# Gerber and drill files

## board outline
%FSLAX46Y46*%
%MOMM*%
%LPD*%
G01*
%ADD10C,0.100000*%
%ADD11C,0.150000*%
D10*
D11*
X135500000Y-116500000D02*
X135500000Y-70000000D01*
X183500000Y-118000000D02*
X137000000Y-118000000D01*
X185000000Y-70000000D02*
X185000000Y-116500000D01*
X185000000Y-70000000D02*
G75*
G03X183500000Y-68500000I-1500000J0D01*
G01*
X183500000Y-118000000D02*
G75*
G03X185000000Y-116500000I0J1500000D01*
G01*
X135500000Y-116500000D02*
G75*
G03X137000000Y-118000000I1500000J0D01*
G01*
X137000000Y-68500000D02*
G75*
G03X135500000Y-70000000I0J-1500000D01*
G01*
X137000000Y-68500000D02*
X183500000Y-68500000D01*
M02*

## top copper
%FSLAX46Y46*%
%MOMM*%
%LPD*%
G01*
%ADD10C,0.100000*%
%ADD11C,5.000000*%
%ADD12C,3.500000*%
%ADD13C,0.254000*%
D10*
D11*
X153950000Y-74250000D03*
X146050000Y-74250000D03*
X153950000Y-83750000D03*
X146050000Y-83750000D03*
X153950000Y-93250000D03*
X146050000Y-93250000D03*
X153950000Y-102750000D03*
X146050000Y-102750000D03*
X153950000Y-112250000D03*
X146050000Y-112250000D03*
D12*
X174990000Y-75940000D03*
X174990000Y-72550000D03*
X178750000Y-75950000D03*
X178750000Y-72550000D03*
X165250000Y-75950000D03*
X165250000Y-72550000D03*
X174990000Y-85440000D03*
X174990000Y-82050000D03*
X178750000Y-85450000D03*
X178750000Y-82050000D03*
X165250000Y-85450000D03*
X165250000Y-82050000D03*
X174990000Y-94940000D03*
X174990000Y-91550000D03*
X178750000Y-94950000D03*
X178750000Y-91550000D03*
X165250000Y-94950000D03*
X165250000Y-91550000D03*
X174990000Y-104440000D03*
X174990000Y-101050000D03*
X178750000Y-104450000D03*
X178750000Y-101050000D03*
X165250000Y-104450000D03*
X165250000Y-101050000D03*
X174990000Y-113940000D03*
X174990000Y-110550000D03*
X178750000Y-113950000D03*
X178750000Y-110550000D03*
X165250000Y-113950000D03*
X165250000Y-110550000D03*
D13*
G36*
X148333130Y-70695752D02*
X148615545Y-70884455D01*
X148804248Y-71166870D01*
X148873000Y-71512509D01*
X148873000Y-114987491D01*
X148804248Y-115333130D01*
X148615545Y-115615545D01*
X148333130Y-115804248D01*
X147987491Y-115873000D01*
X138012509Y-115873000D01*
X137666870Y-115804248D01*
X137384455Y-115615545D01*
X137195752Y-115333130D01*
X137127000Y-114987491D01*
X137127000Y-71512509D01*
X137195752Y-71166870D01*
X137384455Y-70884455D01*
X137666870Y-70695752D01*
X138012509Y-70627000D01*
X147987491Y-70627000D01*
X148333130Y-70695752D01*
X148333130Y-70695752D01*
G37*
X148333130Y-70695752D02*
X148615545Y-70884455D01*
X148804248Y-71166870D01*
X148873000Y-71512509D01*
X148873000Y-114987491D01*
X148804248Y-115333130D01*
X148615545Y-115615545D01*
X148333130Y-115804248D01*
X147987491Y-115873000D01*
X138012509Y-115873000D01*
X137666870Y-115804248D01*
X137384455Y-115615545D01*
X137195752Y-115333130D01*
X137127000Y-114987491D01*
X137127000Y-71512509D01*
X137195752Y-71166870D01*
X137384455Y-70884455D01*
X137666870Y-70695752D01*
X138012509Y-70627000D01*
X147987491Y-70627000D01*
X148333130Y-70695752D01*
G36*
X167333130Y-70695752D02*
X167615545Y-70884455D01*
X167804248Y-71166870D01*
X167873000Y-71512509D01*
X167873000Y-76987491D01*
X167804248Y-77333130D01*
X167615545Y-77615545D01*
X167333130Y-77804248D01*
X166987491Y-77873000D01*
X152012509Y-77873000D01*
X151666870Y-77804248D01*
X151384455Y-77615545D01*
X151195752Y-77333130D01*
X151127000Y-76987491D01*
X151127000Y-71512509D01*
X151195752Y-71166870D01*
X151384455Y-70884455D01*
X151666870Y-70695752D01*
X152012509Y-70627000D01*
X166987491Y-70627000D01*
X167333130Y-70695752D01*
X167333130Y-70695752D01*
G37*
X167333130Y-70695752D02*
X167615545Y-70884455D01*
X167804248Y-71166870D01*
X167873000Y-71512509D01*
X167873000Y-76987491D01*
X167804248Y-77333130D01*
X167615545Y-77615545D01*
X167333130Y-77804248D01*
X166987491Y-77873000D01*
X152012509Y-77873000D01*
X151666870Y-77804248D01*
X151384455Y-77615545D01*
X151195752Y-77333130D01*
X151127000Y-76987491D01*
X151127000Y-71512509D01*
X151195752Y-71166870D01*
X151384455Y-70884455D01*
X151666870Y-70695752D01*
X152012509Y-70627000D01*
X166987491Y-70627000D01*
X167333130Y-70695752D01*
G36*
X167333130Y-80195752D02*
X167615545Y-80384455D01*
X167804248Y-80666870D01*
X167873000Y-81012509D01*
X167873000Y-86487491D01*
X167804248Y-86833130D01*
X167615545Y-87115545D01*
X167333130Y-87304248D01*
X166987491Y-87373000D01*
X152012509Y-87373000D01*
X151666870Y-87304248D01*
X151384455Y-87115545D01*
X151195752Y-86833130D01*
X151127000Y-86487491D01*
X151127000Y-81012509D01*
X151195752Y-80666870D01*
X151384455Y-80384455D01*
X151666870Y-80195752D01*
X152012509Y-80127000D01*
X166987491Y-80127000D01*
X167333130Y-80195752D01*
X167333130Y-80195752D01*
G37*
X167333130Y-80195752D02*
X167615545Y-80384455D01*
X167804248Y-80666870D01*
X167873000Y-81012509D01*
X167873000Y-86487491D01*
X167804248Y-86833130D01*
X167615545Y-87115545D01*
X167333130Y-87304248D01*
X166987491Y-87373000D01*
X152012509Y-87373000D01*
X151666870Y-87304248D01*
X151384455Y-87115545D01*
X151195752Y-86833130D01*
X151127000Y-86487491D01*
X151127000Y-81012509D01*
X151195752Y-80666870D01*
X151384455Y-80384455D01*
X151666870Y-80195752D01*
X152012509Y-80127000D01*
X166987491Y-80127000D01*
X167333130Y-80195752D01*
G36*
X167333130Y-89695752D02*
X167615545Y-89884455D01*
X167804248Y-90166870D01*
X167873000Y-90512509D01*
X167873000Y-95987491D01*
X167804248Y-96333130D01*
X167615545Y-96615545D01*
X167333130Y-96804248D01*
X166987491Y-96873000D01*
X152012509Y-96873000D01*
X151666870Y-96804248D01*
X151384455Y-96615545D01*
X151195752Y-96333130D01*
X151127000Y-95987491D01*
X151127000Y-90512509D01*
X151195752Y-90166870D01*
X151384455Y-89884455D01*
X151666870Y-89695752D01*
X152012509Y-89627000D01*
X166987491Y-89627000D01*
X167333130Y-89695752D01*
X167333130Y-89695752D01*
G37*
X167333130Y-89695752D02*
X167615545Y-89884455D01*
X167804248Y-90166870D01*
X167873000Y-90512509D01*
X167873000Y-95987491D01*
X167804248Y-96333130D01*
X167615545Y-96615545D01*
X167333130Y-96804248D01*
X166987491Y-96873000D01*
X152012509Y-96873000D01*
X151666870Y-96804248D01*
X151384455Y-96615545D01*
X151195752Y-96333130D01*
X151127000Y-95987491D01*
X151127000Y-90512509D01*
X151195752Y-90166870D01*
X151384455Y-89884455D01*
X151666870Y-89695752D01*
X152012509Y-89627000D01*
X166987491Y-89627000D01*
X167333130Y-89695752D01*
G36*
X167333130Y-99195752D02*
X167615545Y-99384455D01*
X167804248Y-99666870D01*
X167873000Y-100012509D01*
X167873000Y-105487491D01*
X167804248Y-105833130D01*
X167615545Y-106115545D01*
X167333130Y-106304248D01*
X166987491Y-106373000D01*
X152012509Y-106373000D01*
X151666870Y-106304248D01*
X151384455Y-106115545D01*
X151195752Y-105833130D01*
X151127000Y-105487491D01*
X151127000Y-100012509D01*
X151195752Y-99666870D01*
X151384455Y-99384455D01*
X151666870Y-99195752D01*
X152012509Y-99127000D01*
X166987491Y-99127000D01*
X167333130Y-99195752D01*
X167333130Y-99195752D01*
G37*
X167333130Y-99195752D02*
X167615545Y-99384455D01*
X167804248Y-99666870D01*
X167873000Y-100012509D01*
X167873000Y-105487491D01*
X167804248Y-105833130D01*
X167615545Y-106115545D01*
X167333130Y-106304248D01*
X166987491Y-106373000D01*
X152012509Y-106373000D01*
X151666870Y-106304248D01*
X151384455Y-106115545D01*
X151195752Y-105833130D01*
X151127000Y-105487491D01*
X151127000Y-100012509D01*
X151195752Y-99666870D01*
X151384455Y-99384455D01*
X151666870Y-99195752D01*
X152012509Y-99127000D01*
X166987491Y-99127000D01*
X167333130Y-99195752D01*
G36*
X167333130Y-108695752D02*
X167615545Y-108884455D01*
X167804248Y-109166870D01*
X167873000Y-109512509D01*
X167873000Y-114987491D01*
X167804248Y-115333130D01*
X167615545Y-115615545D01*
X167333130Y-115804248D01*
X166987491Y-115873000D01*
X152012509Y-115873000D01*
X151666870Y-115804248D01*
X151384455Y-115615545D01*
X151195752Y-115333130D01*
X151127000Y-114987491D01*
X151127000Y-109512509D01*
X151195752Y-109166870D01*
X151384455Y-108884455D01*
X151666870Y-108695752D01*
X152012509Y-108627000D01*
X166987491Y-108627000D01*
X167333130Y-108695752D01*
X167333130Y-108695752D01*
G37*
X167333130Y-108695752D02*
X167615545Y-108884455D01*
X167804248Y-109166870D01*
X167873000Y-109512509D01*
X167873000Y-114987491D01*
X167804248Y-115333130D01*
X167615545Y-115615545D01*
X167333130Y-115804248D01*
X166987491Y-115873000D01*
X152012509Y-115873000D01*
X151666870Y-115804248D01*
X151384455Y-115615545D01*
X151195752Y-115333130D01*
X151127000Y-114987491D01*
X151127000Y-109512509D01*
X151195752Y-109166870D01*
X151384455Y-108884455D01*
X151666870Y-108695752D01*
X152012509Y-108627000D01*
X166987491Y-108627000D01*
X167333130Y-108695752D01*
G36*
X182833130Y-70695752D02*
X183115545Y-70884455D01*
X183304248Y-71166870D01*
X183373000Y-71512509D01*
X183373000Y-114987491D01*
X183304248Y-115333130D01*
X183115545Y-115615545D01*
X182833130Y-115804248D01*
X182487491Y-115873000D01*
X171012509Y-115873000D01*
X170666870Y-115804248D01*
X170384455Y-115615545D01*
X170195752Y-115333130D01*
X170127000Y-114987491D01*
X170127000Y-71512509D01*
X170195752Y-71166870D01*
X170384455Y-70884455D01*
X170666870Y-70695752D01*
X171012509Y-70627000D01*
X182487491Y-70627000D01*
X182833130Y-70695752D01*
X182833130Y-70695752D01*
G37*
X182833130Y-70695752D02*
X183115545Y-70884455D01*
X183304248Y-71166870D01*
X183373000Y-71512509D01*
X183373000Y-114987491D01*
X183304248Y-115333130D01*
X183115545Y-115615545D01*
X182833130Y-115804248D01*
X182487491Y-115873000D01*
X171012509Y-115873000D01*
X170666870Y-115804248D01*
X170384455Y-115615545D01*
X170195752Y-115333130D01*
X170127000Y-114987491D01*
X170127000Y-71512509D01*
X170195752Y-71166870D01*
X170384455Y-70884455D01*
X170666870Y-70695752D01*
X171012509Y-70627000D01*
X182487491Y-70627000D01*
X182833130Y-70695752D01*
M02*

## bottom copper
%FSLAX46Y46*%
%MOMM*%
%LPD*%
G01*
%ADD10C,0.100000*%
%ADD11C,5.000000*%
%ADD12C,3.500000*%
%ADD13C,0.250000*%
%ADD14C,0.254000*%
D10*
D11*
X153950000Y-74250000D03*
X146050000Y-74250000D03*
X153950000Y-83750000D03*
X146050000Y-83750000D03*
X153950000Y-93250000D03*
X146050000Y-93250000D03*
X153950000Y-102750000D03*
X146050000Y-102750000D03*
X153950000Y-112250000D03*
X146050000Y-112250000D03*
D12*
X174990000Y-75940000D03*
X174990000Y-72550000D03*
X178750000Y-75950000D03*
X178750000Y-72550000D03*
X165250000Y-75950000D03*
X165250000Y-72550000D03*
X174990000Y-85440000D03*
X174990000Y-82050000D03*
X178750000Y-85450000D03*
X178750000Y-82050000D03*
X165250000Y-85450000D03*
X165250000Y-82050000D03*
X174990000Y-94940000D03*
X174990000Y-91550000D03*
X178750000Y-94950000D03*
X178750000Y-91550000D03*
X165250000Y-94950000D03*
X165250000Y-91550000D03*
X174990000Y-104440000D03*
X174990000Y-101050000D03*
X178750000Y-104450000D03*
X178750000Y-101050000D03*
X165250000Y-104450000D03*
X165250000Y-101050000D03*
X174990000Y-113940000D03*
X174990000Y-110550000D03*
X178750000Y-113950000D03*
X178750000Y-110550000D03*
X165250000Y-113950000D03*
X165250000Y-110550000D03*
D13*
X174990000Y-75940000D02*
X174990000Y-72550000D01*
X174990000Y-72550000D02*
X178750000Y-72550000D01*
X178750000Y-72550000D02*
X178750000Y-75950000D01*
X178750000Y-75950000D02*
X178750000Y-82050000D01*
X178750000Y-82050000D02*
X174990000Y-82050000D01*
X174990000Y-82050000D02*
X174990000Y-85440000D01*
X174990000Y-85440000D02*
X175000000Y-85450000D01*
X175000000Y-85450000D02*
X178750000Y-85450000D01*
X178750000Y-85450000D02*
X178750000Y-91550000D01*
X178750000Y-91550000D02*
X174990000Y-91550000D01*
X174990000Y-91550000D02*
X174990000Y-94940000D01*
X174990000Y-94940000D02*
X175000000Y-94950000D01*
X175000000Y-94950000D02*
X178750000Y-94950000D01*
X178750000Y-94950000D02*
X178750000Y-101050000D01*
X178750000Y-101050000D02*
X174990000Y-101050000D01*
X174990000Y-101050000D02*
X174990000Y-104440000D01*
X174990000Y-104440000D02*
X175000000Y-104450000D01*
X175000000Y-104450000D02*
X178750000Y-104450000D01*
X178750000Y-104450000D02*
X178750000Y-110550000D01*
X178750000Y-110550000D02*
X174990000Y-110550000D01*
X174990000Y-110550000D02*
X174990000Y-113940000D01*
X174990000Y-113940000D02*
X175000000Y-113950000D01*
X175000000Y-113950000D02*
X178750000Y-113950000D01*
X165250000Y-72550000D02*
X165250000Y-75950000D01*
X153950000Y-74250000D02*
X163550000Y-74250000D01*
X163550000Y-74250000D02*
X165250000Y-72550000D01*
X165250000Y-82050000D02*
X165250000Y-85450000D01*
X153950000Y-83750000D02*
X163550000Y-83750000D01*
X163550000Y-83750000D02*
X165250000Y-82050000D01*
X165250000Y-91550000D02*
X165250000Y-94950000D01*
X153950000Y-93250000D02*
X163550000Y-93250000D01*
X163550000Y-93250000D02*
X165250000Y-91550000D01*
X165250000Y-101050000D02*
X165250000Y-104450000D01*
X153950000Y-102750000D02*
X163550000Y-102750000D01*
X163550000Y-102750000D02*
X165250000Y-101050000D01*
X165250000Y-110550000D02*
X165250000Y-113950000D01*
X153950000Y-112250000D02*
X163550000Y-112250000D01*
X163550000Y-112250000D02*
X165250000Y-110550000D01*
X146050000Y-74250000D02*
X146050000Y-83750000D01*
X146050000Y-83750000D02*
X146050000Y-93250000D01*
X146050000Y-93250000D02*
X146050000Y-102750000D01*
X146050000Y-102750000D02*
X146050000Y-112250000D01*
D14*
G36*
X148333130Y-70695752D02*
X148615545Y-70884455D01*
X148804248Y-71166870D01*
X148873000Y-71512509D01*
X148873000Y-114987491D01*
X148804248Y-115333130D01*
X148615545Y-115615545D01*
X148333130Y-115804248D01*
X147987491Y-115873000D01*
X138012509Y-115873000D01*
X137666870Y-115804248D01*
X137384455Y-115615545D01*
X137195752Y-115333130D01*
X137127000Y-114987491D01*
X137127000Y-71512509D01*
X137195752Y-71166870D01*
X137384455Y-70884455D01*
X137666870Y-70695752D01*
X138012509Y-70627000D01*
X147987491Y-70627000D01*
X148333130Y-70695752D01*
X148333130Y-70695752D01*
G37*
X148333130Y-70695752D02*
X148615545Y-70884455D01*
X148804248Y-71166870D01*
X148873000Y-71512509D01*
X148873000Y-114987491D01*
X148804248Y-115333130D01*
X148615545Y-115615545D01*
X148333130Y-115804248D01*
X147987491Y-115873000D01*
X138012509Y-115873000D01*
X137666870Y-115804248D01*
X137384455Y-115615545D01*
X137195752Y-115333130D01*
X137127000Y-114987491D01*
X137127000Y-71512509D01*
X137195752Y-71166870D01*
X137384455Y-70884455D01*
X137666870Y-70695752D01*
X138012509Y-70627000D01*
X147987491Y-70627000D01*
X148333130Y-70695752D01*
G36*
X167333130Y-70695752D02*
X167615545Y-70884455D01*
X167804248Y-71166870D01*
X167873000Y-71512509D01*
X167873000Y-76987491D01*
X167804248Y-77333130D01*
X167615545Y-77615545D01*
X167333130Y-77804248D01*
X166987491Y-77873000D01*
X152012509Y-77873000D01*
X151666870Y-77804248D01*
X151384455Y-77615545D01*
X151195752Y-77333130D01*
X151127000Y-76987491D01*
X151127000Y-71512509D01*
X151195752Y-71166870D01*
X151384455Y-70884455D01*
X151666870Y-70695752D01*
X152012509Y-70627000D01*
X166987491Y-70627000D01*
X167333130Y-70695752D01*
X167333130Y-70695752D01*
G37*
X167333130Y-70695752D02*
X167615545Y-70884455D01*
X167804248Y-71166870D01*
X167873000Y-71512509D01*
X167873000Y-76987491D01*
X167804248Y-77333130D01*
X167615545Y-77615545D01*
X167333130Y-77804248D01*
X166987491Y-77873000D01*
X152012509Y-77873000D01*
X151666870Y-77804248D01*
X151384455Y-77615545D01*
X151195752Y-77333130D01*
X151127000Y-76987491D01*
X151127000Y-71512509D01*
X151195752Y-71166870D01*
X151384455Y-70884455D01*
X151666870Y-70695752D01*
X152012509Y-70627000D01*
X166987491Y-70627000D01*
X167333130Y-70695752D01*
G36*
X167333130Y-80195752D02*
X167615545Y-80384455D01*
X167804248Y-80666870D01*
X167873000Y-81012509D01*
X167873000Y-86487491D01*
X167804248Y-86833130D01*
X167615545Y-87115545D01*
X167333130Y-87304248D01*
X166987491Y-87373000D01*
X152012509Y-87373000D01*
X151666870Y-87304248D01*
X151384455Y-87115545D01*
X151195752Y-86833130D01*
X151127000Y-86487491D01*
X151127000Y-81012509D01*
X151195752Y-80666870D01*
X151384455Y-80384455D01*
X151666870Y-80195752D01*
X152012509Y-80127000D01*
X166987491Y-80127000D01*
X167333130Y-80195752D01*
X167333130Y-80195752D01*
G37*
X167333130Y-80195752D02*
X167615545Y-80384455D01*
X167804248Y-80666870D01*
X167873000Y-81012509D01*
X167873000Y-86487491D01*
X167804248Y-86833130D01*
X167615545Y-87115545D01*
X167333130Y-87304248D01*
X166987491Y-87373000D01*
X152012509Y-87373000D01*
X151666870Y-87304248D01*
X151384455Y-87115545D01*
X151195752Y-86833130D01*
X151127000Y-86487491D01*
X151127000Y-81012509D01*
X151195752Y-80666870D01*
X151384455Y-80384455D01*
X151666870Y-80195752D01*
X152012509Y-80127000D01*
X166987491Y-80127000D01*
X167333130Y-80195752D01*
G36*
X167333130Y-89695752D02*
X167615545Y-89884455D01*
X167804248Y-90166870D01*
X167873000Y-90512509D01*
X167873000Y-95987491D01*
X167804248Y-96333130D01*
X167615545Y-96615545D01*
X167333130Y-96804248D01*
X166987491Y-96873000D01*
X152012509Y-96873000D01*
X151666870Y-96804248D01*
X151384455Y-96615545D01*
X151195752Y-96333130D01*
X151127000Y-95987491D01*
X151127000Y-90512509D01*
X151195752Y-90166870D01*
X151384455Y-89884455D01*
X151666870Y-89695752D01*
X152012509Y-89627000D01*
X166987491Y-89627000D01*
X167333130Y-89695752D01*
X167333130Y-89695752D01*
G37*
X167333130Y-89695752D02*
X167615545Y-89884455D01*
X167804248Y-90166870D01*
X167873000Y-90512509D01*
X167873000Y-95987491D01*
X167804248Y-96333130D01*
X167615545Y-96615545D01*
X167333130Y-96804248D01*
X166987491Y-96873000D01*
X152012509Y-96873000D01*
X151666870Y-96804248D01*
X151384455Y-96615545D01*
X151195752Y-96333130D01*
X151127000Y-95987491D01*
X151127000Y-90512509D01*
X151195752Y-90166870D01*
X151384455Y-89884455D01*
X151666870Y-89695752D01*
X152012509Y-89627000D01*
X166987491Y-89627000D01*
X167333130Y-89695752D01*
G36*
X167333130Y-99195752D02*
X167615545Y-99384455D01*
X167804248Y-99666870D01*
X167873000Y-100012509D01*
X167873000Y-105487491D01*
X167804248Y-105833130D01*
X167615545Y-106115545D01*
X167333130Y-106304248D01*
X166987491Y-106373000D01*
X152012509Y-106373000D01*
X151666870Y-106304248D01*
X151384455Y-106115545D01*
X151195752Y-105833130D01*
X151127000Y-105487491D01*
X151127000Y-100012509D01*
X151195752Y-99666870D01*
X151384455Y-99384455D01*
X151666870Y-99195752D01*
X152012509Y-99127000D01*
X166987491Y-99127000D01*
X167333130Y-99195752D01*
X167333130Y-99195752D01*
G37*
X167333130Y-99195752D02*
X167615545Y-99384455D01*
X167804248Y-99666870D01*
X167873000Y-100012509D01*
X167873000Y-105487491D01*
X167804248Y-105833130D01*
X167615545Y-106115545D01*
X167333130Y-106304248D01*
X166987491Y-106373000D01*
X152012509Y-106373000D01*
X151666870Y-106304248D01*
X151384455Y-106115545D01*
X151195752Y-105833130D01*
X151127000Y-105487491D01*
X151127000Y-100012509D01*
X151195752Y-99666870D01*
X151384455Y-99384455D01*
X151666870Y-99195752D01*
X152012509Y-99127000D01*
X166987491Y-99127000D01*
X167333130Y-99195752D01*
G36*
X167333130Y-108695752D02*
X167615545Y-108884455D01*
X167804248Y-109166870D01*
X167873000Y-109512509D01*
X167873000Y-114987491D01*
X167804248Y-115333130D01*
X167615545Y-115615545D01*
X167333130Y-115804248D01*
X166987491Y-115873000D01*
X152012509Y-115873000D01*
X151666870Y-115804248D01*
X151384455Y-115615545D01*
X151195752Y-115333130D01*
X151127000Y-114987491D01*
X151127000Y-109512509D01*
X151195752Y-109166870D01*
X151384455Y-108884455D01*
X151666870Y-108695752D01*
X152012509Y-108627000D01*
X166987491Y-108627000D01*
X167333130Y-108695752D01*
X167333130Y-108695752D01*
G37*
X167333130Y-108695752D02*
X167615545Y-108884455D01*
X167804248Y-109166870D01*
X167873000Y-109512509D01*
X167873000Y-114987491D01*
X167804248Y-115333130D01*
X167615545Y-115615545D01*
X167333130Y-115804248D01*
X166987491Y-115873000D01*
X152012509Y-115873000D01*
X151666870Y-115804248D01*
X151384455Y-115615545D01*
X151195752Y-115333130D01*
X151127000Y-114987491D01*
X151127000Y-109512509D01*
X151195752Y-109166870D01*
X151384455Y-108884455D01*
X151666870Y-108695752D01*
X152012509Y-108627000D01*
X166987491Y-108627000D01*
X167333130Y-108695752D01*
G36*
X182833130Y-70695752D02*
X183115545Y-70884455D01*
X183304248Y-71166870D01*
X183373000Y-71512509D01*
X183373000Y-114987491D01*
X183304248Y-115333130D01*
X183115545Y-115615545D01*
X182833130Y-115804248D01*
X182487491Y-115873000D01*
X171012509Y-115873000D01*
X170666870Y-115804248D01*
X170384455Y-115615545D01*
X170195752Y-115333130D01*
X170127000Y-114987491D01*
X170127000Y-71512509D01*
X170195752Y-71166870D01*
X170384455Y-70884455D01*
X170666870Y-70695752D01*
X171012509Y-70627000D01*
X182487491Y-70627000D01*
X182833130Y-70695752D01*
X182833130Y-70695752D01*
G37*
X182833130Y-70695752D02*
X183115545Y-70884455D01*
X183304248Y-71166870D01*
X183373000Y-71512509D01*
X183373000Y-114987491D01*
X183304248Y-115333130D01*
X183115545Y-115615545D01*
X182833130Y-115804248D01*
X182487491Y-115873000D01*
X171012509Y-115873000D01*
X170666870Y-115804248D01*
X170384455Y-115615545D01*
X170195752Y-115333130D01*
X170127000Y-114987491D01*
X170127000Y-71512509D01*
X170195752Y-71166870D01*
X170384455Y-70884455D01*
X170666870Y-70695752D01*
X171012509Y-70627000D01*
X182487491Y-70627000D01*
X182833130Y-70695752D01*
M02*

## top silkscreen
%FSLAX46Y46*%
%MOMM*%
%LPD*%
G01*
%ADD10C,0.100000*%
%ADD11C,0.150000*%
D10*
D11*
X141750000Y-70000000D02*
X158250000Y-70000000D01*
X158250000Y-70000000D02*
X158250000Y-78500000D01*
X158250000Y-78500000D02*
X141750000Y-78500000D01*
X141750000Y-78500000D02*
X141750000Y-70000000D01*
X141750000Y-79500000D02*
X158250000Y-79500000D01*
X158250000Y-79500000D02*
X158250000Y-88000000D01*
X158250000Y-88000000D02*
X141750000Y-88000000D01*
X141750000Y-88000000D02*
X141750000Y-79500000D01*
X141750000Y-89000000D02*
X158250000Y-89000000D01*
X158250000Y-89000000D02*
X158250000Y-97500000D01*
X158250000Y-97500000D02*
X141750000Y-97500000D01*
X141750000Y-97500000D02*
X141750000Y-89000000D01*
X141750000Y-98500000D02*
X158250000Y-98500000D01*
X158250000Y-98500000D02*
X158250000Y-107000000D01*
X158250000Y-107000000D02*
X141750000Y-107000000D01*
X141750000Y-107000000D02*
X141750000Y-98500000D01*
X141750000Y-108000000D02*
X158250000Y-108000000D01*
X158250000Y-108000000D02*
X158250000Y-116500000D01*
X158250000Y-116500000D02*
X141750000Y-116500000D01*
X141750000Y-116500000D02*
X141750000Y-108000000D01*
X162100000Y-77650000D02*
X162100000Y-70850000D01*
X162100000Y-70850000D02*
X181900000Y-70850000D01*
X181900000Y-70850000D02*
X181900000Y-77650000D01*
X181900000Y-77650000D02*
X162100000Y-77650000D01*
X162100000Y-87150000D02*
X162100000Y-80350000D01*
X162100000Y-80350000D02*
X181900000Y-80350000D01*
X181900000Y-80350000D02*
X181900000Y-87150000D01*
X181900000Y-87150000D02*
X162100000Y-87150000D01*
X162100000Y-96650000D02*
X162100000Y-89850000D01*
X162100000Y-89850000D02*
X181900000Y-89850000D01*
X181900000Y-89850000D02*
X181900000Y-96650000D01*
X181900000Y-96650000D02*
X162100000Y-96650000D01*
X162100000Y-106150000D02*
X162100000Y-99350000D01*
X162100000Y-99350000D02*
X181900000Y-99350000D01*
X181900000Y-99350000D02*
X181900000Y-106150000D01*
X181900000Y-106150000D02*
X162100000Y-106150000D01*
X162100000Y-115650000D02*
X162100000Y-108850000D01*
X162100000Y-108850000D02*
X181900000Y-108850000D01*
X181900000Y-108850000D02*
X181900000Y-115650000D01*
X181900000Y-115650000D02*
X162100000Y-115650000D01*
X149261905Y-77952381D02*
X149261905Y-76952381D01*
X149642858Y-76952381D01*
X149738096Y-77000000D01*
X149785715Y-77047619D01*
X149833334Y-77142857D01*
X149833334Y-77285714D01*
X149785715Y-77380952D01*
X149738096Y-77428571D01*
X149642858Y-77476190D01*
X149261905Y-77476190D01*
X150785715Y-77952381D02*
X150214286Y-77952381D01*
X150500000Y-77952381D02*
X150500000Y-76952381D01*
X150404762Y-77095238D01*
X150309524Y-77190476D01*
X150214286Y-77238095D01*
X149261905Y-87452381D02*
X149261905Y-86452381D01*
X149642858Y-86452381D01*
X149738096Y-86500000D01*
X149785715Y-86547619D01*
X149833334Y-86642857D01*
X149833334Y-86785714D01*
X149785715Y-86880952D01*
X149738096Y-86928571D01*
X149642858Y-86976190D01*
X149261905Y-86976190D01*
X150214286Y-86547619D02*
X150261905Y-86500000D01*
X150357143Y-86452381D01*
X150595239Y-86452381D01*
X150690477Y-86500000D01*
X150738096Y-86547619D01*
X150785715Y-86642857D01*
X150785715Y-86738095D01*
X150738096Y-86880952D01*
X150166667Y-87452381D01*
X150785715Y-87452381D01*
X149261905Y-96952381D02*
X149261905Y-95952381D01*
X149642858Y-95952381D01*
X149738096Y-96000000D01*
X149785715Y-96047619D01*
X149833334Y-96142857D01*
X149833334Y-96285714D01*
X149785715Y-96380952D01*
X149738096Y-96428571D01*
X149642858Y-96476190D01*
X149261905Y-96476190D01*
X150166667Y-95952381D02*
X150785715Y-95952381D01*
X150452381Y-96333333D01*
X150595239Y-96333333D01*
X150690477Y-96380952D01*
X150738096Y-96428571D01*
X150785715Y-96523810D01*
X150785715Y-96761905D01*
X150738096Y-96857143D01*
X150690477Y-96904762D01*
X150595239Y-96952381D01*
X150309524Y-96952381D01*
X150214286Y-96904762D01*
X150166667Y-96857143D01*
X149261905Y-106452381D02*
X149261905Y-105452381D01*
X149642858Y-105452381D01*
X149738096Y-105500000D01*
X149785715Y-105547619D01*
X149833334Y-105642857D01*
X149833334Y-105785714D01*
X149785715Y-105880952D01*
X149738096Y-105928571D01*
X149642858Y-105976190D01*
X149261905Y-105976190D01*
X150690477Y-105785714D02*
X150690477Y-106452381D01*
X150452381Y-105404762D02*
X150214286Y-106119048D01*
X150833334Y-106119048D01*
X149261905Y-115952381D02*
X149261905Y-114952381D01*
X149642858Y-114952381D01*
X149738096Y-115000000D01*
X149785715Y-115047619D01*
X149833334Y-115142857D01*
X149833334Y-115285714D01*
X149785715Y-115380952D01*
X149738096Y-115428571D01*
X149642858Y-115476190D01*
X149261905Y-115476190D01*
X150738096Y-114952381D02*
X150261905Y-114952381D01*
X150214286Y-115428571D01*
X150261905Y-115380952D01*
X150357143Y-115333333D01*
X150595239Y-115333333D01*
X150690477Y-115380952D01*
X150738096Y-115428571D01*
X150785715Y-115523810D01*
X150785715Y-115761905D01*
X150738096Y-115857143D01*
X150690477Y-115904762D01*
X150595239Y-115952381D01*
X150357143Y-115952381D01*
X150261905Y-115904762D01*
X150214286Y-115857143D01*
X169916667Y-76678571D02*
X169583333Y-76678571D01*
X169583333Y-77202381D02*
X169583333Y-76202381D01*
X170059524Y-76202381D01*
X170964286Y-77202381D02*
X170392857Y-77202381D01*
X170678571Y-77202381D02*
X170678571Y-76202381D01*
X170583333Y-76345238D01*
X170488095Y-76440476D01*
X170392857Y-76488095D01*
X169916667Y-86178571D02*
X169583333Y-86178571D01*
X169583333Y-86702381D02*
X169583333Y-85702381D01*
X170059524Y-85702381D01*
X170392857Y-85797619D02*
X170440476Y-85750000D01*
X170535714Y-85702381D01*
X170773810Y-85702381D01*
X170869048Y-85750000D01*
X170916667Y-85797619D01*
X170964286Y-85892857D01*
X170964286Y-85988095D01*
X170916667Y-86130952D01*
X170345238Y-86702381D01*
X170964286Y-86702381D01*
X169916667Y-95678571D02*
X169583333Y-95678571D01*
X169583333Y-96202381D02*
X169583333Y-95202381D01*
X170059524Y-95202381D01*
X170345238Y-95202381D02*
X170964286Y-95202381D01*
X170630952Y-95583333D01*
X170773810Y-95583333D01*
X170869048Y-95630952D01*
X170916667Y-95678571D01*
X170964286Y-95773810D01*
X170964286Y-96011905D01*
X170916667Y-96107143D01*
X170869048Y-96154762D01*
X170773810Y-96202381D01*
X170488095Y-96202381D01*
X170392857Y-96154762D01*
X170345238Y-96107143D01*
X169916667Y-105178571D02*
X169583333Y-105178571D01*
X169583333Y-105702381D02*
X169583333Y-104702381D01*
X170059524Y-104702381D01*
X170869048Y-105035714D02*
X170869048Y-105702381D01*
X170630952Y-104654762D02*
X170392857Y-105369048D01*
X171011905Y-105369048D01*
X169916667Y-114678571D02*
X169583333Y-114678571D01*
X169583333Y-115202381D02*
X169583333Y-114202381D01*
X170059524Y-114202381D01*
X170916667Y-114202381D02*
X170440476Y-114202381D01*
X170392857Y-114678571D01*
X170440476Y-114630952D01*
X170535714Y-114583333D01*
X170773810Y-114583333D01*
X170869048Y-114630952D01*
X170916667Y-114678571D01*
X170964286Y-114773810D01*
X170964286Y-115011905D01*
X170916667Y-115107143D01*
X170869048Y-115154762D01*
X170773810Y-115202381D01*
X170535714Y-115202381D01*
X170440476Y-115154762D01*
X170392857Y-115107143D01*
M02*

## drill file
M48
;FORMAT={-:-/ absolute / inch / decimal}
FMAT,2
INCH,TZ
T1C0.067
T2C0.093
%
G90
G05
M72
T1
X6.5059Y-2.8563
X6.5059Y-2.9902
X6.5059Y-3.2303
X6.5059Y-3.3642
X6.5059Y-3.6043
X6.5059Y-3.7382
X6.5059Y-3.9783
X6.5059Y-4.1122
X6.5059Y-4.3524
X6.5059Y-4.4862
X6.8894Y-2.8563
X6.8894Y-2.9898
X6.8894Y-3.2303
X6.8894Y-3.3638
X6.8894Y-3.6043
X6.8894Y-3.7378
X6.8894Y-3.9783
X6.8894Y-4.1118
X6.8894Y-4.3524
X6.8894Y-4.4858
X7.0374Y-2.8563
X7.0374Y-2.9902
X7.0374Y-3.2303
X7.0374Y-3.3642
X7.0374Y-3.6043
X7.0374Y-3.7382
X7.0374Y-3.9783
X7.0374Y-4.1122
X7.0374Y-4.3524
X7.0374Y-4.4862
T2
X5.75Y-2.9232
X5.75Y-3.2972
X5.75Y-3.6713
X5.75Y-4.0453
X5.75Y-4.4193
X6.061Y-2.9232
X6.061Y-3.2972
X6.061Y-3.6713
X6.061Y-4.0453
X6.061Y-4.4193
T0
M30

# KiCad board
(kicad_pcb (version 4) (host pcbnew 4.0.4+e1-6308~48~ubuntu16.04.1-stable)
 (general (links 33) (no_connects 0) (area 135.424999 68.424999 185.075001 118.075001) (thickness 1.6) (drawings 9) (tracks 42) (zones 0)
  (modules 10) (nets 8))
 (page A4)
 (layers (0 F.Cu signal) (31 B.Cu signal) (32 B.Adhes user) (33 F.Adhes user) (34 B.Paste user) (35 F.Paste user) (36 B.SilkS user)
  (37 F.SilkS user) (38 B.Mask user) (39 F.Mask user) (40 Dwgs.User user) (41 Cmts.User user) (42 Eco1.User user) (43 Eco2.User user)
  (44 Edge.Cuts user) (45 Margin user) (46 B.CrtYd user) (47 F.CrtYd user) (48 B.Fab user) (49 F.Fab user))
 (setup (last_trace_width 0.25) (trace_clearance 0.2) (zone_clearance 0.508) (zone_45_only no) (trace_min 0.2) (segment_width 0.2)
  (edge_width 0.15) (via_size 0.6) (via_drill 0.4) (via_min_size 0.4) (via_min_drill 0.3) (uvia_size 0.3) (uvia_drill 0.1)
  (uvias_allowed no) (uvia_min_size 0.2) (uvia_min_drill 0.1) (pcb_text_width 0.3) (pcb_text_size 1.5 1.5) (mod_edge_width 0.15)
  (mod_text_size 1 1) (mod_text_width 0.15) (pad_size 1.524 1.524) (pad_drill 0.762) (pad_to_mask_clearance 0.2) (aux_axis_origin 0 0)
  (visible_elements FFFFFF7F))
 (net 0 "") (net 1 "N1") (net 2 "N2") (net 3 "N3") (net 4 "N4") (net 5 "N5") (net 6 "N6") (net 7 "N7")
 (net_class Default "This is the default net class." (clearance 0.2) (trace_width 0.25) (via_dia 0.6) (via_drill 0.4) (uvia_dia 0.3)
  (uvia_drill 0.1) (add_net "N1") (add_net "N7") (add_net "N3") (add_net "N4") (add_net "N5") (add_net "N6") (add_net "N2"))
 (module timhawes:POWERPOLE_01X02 (layer F.Cu) (at 150 74.25)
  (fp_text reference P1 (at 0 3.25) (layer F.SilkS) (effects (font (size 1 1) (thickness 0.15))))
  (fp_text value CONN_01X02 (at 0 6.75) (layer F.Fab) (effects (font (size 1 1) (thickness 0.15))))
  (fp_line (start -8.25 -4.25) (end 8.25 -4.25) (layer F.SilkS) (width 0.15))
  (fp_line (start 8.25 -4.25) (end 8.25 4.25) (layer F.SilkS) (width 0.15))
  (fp_line (start 8.25 4.25) (end -8.25 4.25) (layer F.SilkS) (width 0.15))
  (fp_line (start -8.25 4.25) (end -8.25 -4.25) (layer F.SilkS) (width 0.15))
  (pad 2 thru_hole circle (at 3.95 0) (size 5 5) (drill 2.35) (layers *.Cu *.Mask) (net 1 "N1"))
  (pad 1 thru_hole circle (at -3.95 0) (size 5 5) (drill 2.35) (layers *.Cu *.Mask) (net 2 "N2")))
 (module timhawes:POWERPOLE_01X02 (layer F.Cu) (at 150 83.75)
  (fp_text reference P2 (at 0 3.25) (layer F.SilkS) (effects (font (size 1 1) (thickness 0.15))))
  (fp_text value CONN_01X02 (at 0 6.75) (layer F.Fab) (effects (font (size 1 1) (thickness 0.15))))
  (fp_line (start -8.25 -4.25) (end 8.25 -4.25) (layer F.SilkS) (width 0.15))
  (fp_line (start 8.25 -4.25) (end 8.25 4.25) (layer F.SilkS) (width 0.15))
  (fp_line (start 8.25 4.25) (end -8.25 4.25) (layer F.SilkS) (width 0.15))
  (fp_line (start -8.25 4.25) (end -8.25 -4.25) (layer F.SilkS) (width 0.15))
  (pad 2 thru_hole circle (at 3.95 0) (size 5 5) (drill 2.35) (layers *.Cu *.Mask) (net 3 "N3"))
  (pad 1 thru_hole circle (at -3.95 0) (size 5 5) (drill 2.35) (layers *.Cu *.Mask) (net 2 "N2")))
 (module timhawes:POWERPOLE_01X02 (layer F.Cu) (at 150 93.25)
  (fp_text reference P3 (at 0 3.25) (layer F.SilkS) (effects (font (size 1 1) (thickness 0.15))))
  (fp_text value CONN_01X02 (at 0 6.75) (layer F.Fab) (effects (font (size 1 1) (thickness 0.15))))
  (fp_line (start -8.25 -4.25) (end 8.25 -4.25) (layer F.SilkS) (width 0.15))
  (fp_line (start 8.25 -4.25) (end 8.25 4.25) (layer F.SilkS) (width 0.15))
  (fp_line (start 8.25 4.25) (end -8.25 4.25) (layer F.SilkS) (width 0.15))
  (fp_line (start -8.25 4.25) (end -8.25 -4.25) (layer F.SilkS) (width 0.15))
  (pad 2 thru_hole circle (at 3.95 0) (size 5 5) (drill 2.35) (layers *.Cu *.Mask) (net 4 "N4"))
  (pad 1 thru_hole circle (at -3.95 0) (size 5 5) (drill 2.35) (layers *.Cu *.Mask) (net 2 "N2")))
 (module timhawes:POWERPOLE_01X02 (layer F.Cu) (at 150 102.75)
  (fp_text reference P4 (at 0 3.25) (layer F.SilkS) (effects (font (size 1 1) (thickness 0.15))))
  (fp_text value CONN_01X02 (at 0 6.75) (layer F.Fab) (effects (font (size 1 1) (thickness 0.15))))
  (fp_line (start -8.25 -4.25) (end 8.25 -4.25) (layer F.SilkS) (width 0.15))
  (fp_line (start 8.25 -4.25) (end 8.25 4.25) (layer F.SilkS) (width 0.15))
  (fp_line (start 8.25 4.25) (end -8.25 4.25) (layer F.SilkS) (width 0.15))
  (fp_line (start -8.25 4.25) (end -8.25 -4.25) (layer F.SilkS) (width 0.15))
  (pad 2 thru_hole circle (at 3.95 0) (size 5 5) (drill 2.35) (layers *.Cu *.Mask) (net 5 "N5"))
  (pad 1 thru_hole circle (at -3.95 0) (size 5 5) (drill 2.35) (layers *.Cu *.Mask) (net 2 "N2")))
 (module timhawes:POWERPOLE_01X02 (layer F.Cu) (at 150 112.25)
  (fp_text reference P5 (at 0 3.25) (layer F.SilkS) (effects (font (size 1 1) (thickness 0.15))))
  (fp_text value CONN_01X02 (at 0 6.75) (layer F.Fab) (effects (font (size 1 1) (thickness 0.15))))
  (fp_line (start -8.25 -4.25) (end 8.25 -4.25) (layer F.SilkS) (width 0.15))
  (fp_line (start 8.25 -4.25) (end 8.25 4.25) (layer F.SilkS) (width 0.15))
  (fp_line (start 8.25 4.25) (end -8.25 4.25) (layer F.SilkS) (width 0.15))
  (fp_line (start -8.25 4.25) (end -8.25 -4.25) (layer F.SilkS) (width 0.15))
  (pad 2 thru_hole circle (at 3.95 0) (size 5 5) (drill 2.35) (layers *.Cu *.Mask) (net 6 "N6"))
  (pad 1 thru_hole circle (at -3.95 0) (size 5 5) (drill 2.35) (layers *.Cu *.Mask) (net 2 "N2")))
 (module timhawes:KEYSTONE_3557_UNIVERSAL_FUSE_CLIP (layer F.Cu) (at 172 74.25)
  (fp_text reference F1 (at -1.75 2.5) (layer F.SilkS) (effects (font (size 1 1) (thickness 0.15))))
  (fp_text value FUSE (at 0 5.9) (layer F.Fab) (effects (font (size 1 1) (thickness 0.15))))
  (fp_line (start -9.9 3.4) (end -9.9 -3.4) (layer F.SilkS) (width 0.15))
  (fp_line (start -9.9 -3.4) (end 9.9 -3.4) (layer F.SilkS) (width 0.15))
  (fp_line (start 9.9 -3.4) (end 9.9 3.4) (layer F.SilkS) (width 0.15))
  (fp_line (start 9.9 3.4) (end -9.9 3.4) (layer F.SilkS) (width 0.15))
  (pad 2 thru_hole circle (at 2.99 1.69) (size 3.5 3.5) (drill 1.7) (layers *.Cu *.Mask) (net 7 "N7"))
  (pad 2 thru_hole circle (at 2.99 -1.7) (size 3.5 3.5) (drill 1.7) (layers *.Cu *.Mask) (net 7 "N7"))
  (pad 2 thru_hole circle (at 6.75 1.7) (size 3.5 3.5) (drill 1.7) (layers *.Cu *.Mask) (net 7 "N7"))
  (pad 2 thru_hole circle (at 6.75 -1.7) (size 3.5 3.5) (drill 1.7) (layers *.Cu *.Mask) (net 7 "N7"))
  (pad 1 thru_hole circle (at -6.75 1.7) (size 3.5 3.5) (drill 1.7) (layers *.Cu *.Mask) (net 1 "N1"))
  (pad 1 thru_hole circle (at -6.75 -1.7) (size 3.5 3.5) (drill 1.7) (layers *.Cu *.Mask) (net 1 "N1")))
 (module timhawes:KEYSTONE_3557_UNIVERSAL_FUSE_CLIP (layer F.Cu) (at 172 83.75)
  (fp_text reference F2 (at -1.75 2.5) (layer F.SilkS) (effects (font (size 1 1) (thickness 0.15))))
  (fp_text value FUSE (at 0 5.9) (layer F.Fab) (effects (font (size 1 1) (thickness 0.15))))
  (fp_line (start -9.9 3.4) (end -9.9 -3.4) (layer F.SilkS) (width 0.15))
  (fp_line (start -9.9 -3.4) (end 9.9 -3.4) (layer F.SilkS) (width 0.15))
  (fp_line (start 9.9 -3.4) (end 9.9 3.4) (layer F.SilkS) (width 0.15))
  (fp_line (start 9.9 3.4) (end -9.9 3.4) (layer F.SilkS) (width 0.15))
  (pad 2 thru_hole circle (at 2.99 1.69) (size 3.5 3.5) (drill 1.7) (layers *.Cu *.Mask) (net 7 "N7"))
  (pad 2 thru_hole circle (at 2.99 -1.7) (size 3.5 3.5) (drill 1.7) (layers *.Cu *.Mask) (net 7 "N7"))
  (pad 2 thru_hole circle (at 6.75 1.7) (size 3.5 3.5) (drill 1.7) (layers *.Cu *.Mask) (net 7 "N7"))
  (pad 2 thru_hole circle (at 6.75 -1.7) (size 3.5 3.5) (drill 1.7) (layers *.Cu *.Mask) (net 7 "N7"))
  (pad 1 thru_hole circle (at -6.75 1.7) (size 3.5 3.5) (drill 1.7) (layers *.Cu *.Mask) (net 3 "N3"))
  (pad 1 thru_hole circle (at -6.75 -1.7) (size 3.5 3.5) (drill 1.7) (layers *.Cu *.Mask) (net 3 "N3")))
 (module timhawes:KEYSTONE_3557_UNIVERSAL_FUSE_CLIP (layer F.Cu) (at 172 93.25)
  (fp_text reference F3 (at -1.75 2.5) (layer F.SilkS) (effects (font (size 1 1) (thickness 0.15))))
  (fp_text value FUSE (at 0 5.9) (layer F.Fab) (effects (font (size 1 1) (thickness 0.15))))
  (fp_line (start -9.9 3.4) (end -9.9 -3.4) (layer F.SilkS) (width 0.15))
  (fp_line (start -9.9 -3.4) (end 9.9 -3.4) (layer F.SilkS) (width 0.15))
  (fp_line (start 9.9 -3.4) (end 9.9 3.4) (layer F.SilkS) (width 0.15))
  (fp_line (start 9.9 3.4) (end -9.9 3.4) (layer F.SilkS) (width 0.15))
  (pad 2 thru_hole circle (at 2.99 1.69) (size 3.5 3.5) (drill 1.7) (layers *.Cu *.Mask) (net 7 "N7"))
  (pad 2 thru_hole circle (at 2.99 -1.7) (size 3.5 3.5) (drill 1.7) (layers *.Cu *.Mask) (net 7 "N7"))
  (pad 2 thru_hole circle (at 6.75 1.7) (size 3.5 3.5) (drill 1.7) (layers *.Cu *.Mask) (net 7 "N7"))
  (pad 2 thru_hole circle (at 6.75 -1.7) (size 3.5 3.5) (drill 1.7) (layers *.Cu *.Mask) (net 7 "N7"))
  (pad 1 thru_hole circle (at -6.75 1.7) (size 3.5 3.5) (drill 1.7) (layers *.Cu *.Mask) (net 4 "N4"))
  (pad 1 thru_hole circle (at -6.75 -1.7) (size 3.5 3.5) (drill 1.7) (layers *.Cu *.Mask) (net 4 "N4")))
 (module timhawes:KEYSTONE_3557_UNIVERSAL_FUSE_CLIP (layer F.Cu) (at 172 102.75)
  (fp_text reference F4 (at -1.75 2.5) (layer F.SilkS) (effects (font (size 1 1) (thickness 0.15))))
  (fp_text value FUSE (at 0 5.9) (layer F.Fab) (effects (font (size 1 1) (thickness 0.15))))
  (fp_line (start -9.9 3.4) (end -9.9 -3.4) (layer F.SilkS) (width 0.15))
  (fp_line (start -9.9 -3.4) (end 9.9 -3.4) (layer F.SilkS) (width 0.15))
  (fp_line (start 9.9 -3.4) (end 9.9 3.4) (layer F.SilkS) (width 0.15))
  (fp_line (start 9.9 3.4) (end -9.9 3.4) (layer F.SilkS) (width 0.15))
  (pad 2 thru_hole circle (at 2.99 1.69) (size 3.5 3.5) (drill 1.7) (layers *.Cu *.Mask) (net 7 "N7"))
  (pad 2 thru_hole circle (at 2.99 -1.7) (size 3.5 3.5) (drill 1.7) (layers *.Cu *.Mask) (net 7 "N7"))
  (pad 2 thru_hole circle (at 6.75 1.7) (size 3.5 3.5) (drill 1.7) (layers *.Cu *.Mask) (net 7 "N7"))
  (pad 2 thru_hole circle (at 6.75 -1.7) (size 3.5 3.5) (drill 1.7) (layers *.Cu *.Mask) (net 7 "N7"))
  (pad 1 thru_hole circle (at -6.75 1.7) (size 3.5 3.5) (drill 1.7) (layers *.Cu *.Mask) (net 5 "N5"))
  (pad 1 thru_hole circle (at -6.75 -1.7) (size 3.5 3.5) (drill 1.7) (layers *.Cu *.Mask) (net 5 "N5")))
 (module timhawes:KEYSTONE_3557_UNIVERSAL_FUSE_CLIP (layer F.Cu) (at 172 112.25)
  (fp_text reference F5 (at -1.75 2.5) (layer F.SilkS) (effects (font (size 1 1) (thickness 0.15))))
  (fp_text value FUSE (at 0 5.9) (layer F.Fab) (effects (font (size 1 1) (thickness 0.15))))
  (fp_line (start -9.9 3.4) (end -9.9 -3.4) (layer F.SilkS) (width 0.15))
  (fp_line (start -9.9 -3.4) (end 9.9 -3.4) (layer F.SilkS) (width 0.15))
  (fp_line (start 9.9 -3.4) (end 9.9 3.4) (layer F.SilkS) (width 0.15))
  (fp_line (start 9.9 3.4) (end -9.9 3.4) (layer F.SilkS) (width 0.15))
  (pad 2 thru_hole circle (at 2.99 1.69) (size 3.5 3.5) (drill 1.7) (layers *.Cu *.Mask) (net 7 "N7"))
  (pad 2 thru_hole circle (at 2.99 -1.7) (size 3.5 3.5) (drill 1.7) (layers *.Cu *.Mask) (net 7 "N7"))
  (pad 2 thru_hole circle (at 6.75 1.7) (size 3.5 3.5) (drill 1.7) (layers *.Cu *.Mask) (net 7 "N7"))
  (pad 2 thru_hole circle (at 6.75 -1.7) (size 3.5 3.5) (drill 1.7) (layers *.Cu *.Mask) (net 7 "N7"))
  (pad 1 thru_hole circle (at -6.75 1.7) (size 3.5 3.5) (drill 1.7) (layers *.Cu *.Mask) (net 6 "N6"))
  (pad 1 thru_hole circle (at -6.75 -1.7) (size 3.5 3.5) (drill 1.7) (layers *.Cu *.Mask) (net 6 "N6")))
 (gr_line (start 135.5 116.5) (end 135.5 70) (angle 90) (layer Edge.Cuts) (width 0.15))
 (gr_line (start 183.5 118) (end 137 118) (angle 90) (layer Edge.Cuts) (width 0.15))
 (gr_line (start 185 70) (end 185 116.5) (angle 90) (layer Edge.Cuts) (width 0.15))
 (gr_arc (start 183.5 70) (end 183.5 68.5) (angle 90) (layer Edge.Cuts) (width 0.15))
 (gr_arc (start 183.5 116.5) (end 185 116.5) (angle 90) (layer Edge.Cuts) (width 0.15))
 (gr_arc (start 137 116.5) (end 137 118) (angle 90) (layer Edge.Cuts) (width 0.15))
 (gr_arc (start 137 70) (end 135.5 70) (angle 90) (layer Edge.Cuts) (width 0.15))
 (gr_line (start 137 68.5) (end 183.5 68.5) (angle 90) (layer Edge.Cuts) (width 0.15))
 (segment (start 174.99 75.94) (end 174.99 72.55) (width 0.25) (layer B.Cu) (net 7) (status C00000))
 (segment (start 174.99 72.55) (end 178.75 72.55) (width 0.25) (layer B.Cu) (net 7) (status C00000))
 (segment (start 178.75 72.55) (end 178.75 75.95) (width 0.25) (layer B.Cu) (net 7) (status C00000))
 (segment (start 178.75 75.95) (end 178.75 82.05) (width 0.25) (layer B.Cu) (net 7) (status C00000))
 (segment (start 178.75 82.05) (end 174.99 82.05) (width 0.25) (layer B.Cu) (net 7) (status C00000))
 (segment (start 174.99 82.05) (end 174.99 85.44) (width 0.25) (layer B.Cu) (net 7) (status C00000))
 (segment (start 174.99 85.44) (end 175 85.45) (width 0.25) (layer B.Cu) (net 7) (status C00000))
 (segment (start 175 85.45) (end 178.75 85.45) (width 0.25) (layer B.Cu) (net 7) (status C00000))
 (segment (start 178.75 85.45) (end 178.75 91.55) (width 0.25) (layer B.Cu) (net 7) (status C00000))
 (segment (start 178.75 91.55) (end 174.99 91.55) (width 0.25) (layer B.Cu) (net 7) (status C00000))
 (segment (start 174.99 91.55) (end 174.99 94.94) (width 0.25) (layer B.Cu) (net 7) (status C00000))
 (segment (start 174.99 94.94) (end 175 94.95) (width 0.25) (layer B.Cu) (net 7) (status C00000))
 (segment (start 175 94.95) (end 178.75 94.95) (width 0.25) (layer B.Cu) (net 7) (status C00000))
 (segment (start 178.75 94.95) (end 178.75 101.05) (width 0.25) (layer B.Cu) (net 7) (status C00000))
 (segment (start 178.75 101.05) (end 174.99 101.05) (width 0.25) (layer B.Cu) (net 7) (status C00000))
 (segment (start 174.99 101.05) (end 174.99 104.44) (width 0.25) (layer B.Cu) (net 7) (status C00000))
 (segment (start 174.99 104.44) (end 175 104.45) (width 0.25) (layer B.Cu) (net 7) (status C00000))
 (segment (start 175 104.45) (end 178.75 104.45) (width 0.25) (layer B.Cu) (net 7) (status C00000))
 (segment (start 178.75 104.45) (end 178.75 110.55) (width 0.25) (layer B.Cu) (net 7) (status C00000))
 (segment (start 178.75 110.55) (end 174.99 110.55) (width 0.25) (layer B.Cu) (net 7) (status C00000))
 (segment (start 174.99 110.55) (end 174.99 113.94) (width 0.25) (layer B.Cu) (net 7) (status C00000))
 (segment (start 174.99 113.94) (end 175 113.95) (width 0.25) (layer B.Cu) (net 7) (status C00000))
 (segment (start 175 113.95) (end 178.75 113.95) (width 0.25) (layer B.Cu) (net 7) (status C00000))
 (segment (start 165.25 72.55) (end 165.25 75.95) (width 0.25) (layer B.Cu) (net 1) (status C00000))
 (segment (start 153.95 74.25) (end 163.55 74.25) (width 0.25) (layer B.Cu) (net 1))
 (segment (start 163.55 74.25) (end 165.25 72.55) (width 0.25) (layer B.Cu) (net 1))
 (segment (start 165.25 82.05) (end 165.25 85.45) (width 0.25) (layer B.Cu) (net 3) (status C00000))
 (segment (start 153.95 83.75) (end 163.55 83.75) (width 0.25) (layer B.Cu) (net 3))
 (segment (start 163.55 83.75) (end 165.25 82.05) (width 0.25) (layer B.Cu) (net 3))
 (segment (start 165.25 91.55) (end 165.25 94.95) (width 0.25) (layer B.Cu) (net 4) (status C00000))
 (segment (start 153.95 93.25) (end 163.55 93.25) (width 0.25) (layer B.Cu) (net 4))
 (segment (start 163.55 93.25) (end 165.25 91.55) (width 0.25) (layer B.Cu) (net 4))
 (segment (start 165.25 101.05) (end 165.25 104.45) (width 0.25) (layer B.Cu) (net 5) (status C00000))
 (segment (start 153.95 102.75) (end 163.55 102.75) (width 0.25) (layer B.Cu) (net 5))
 (segment (start 163.55 102.75) (end 165.25 101.05) (width 0.25) (layer B.Cu) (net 5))
 (segment (start 165.25 110.55) (end 165.25 113.95) (width 0.25) (layer B.Cu) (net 6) (status C00000))
 (segment (start 153.95 112.25) (end 163.55 112.25) (width 0.25) (layer B.Cu) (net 6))
 (segment (start 163.55 112.25) (end 165.25 110.55) (width 0.25) (layer B.Cu) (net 6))
 (segment (start 146.05 74.25) (end 146.05 83.75) (width 0.25) (layer B.Cu) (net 2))
 (segment (start 146.05 83.75) (end 146.05 93.25) (width 0.25) (layer B.Cu) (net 2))
 (segment (start 146.05 93.25) (end 146.05 102.75) (width 0.25) (layer B.Cu) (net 2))
 (segment (start 146.05 102.75) (end 146.05 112.25) (width 0.25) (layer B.Cu) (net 2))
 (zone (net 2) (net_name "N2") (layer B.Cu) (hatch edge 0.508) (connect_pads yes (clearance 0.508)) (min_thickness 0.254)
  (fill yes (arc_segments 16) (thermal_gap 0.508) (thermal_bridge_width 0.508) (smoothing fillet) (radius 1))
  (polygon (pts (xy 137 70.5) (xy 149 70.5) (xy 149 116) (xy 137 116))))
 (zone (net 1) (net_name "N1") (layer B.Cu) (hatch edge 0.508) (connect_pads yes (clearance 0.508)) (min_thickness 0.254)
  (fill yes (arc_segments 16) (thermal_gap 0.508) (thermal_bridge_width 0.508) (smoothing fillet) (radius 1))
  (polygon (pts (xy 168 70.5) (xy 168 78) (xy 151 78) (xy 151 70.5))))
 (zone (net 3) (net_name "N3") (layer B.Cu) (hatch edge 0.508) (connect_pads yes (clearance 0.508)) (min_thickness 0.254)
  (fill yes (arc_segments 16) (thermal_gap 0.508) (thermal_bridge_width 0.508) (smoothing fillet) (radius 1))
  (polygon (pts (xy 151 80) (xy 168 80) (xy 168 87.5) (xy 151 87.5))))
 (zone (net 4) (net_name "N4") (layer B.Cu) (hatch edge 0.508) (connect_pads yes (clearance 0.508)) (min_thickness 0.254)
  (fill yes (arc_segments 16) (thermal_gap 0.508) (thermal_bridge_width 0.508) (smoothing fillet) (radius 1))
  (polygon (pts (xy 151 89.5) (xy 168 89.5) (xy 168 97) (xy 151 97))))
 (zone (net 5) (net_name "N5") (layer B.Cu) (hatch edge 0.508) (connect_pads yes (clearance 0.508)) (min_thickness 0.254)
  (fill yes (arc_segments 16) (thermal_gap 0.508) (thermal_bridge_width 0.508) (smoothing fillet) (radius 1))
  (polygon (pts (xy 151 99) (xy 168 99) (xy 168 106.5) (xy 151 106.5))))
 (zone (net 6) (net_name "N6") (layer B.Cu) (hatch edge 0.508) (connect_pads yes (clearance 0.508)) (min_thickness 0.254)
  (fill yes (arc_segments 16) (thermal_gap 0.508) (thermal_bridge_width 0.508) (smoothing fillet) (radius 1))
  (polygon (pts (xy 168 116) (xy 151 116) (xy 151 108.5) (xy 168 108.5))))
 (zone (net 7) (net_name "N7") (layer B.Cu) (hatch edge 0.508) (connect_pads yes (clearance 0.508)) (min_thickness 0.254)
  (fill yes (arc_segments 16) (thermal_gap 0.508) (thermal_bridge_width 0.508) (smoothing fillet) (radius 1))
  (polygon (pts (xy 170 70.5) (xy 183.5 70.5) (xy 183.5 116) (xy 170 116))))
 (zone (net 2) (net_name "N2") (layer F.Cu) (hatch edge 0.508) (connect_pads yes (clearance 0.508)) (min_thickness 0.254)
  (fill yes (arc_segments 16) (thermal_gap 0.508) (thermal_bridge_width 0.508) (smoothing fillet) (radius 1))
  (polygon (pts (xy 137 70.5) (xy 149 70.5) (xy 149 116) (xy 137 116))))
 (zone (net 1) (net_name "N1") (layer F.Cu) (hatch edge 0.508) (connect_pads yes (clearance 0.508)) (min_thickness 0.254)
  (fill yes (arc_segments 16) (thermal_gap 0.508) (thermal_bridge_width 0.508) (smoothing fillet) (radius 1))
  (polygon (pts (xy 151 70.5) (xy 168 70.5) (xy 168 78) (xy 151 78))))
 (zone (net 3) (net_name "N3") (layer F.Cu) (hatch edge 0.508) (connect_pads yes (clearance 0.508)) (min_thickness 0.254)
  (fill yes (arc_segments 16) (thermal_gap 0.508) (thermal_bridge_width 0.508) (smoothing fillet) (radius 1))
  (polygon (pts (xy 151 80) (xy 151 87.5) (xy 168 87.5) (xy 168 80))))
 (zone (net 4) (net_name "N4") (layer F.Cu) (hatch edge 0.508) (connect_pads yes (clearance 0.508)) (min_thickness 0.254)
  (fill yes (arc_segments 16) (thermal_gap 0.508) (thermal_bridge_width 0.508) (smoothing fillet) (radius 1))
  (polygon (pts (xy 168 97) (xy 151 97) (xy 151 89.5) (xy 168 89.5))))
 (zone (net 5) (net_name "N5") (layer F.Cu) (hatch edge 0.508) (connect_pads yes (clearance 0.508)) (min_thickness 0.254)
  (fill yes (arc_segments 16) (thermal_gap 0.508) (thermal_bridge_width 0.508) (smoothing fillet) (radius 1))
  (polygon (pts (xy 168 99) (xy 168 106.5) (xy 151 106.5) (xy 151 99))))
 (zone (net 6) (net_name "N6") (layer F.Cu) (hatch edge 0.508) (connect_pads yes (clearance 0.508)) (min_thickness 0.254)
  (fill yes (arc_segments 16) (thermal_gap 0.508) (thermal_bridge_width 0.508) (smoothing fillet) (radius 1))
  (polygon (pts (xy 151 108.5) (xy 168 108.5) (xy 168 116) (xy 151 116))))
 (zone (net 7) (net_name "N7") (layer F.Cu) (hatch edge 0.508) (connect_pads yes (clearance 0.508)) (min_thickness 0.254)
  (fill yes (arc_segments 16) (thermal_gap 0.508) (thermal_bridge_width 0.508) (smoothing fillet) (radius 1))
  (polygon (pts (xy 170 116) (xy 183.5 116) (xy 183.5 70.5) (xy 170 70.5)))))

